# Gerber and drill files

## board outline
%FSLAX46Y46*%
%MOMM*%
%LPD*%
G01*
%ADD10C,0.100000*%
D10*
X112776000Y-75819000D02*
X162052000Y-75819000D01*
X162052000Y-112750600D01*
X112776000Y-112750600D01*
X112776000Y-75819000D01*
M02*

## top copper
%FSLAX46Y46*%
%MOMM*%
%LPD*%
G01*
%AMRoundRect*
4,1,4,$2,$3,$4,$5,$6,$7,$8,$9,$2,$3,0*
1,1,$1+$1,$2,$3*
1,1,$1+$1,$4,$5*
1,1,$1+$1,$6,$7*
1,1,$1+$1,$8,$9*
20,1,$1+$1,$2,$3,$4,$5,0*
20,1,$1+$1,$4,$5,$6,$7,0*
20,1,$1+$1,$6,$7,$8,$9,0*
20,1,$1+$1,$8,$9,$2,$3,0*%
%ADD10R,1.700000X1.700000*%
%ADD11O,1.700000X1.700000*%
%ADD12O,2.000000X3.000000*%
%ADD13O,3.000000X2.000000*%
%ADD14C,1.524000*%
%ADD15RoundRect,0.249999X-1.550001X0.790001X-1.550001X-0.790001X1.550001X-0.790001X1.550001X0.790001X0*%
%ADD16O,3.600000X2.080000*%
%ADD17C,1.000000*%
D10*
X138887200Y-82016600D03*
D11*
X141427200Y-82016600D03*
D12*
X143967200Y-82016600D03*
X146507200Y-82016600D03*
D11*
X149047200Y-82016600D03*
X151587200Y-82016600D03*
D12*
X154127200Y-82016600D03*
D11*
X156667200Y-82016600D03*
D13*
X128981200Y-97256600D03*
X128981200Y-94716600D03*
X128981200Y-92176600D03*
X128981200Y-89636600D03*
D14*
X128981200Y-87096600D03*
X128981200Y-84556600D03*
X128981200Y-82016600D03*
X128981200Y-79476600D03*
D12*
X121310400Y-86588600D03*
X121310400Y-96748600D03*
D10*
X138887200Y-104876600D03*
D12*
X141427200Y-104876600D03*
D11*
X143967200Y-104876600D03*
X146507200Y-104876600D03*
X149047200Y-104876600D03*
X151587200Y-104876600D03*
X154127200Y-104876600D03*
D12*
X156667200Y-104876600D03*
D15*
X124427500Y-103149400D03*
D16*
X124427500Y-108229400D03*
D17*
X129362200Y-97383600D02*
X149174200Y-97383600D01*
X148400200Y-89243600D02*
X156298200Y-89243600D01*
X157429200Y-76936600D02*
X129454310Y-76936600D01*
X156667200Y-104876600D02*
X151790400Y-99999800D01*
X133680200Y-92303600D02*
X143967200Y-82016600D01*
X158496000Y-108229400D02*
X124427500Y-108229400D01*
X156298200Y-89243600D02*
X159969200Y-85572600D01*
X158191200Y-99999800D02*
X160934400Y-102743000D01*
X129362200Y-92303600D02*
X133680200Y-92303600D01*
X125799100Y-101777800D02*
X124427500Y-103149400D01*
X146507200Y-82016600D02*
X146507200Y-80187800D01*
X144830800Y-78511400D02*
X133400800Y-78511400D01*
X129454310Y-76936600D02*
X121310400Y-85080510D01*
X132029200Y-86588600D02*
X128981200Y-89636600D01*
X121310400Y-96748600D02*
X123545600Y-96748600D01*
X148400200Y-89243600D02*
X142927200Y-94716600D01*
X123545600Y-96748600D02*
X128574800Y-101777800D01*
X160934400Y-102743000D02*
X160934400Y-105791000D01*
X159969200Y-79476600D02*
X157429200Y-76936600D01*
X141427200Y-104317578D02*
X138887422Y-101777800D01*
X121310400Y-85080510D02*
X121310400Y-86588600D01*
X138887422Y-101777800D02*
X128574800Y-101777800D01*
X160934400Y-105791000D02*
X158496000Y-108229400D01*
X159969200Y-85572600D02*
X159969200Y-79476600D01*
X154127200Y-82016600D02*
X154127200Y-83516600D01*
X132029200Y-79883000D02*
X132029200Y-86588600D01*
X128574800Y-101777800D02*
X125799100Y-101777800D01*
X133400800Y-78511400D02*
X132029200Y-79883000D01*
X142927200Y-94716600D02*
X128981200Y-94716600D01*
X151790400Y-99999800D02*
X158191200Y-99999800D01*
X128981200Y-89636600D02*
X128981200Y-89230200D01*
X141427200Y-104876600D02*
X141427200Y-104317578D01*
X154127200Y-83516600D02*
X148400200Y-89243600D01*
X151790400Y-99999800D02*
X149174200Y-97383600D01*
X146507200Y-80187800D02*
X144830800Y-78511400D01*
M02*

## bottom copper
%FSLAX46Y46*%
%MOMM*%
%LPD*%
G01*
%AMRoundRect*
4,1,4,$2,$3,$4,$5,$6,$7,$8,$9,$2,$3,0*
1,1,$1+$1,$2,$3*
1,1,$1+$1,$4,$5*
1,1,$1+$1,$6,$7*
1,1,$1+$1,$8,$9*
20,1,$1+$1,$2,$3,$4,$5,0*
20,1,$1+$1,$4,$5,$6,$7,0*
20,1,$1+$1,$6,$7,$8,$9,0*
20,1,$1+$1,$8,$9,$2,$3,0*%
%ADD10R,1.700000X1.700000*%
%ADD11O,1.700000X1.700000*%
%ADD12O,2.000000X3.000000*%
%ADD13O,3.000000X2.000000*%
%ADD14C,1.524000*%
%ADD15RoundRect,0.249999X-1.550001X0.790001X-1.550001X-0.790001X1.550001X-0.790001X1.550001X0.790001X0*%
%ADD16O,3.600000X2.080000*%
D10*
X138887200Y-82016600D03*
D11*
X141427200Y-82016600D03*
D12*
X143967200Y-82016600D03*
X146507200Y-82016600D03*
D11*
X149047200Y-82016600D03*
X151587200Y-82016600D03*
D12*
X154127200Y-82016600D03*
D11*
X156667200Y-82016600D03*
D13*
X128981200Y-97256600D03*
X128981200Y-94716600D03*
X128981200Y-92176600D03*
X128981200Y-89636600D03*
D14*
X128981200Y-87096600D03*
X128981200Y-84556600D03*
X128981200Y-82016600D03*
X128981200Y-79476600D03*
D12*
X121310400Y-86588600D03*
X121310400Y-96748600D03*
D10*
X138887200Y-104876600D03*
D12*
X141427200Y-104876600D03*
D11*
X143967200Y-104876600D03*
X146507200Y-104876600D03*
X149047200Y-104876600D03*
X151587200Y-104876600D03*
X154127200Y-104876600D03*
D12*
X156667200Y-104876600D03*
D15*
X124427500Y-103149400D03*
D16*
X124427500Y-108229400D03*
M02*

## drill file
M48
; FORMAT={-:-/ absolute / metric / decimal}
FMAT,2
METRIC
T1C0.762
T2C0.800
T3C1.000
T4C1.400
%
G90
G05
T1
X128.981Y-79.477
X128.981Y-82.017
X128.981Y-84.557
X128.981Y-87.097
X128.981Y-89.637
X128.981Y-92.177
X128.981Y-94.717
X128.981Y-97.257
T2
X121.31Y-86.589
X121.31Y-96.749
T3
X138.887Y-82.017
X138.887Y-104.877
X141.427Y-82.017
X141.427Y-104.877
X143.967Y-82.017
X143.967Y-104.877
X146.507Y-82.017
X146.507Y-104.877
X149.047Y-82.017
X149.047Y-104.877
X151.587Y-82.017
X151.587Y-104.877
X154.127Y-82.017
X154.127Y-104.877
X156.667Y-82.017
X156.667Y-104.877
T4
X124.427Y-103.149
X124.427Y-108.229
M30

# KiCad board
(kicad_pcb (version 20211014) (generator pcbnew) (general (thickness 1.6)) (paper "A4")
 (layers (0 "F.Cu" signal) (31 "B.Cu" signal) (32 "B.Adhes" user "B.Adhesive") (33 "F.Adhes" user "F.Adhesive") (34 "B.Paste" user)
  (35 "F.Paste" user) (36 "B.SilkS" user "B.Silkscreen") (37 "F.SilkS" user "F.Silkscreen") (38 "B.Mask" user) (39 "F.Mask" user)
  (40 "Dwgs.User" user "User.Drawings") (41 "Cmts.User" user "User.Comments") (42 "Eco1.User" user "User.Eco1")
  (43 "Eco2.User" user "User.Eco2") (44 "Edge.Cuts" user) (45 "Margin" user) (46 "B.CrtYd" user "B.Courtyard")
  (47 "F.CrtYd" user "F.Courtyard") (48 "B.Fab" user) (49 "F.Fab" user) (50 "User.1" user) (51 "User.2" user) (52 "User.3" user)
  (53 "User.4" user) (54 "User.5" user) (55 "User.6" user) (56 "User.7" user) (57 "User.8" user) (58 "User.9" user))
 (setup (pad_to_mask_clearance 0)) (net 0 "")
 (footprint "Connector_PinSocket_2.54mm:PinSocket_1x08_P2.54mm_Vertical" (layer "F.Cu") (at 138.8872 82.0166 90)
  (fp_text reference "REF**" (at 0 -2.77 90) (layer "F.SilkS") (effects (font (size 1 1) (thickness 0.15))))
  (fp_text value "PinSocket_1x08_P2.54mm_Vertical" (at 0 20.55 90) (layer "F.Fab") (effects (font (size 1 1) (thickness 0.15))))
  (pad "1" thru_hole rect (at 0 0 90) (size 1.7 1.7) (drill 1) (layers *.Cu *.Mask))
  (pad "2" thru_hole oval (at 0 2.54 90) (size 1.7 1.7) (drill 1) (layers *.Cu *.Mask))
  (pad "3" thru_hole oval (at 0 5.08 90) (size 3 2) (drill 1) (layers *.Cu *.Mask))
  (pad "4" thru_hole oval (at 0 7.62 90) (size 3 2) (drill 1) (layers *.Cu *.Mask))
  (pad "5" thru_hole oval (at 0 10.16 90) (size 1.7 1.7) (drill 1) (layers *.Cu *.Mask))
  (pad "6" thru_hole oval (at 0 12.7 90) (size 1.7 1.7) (drill 1) (layers *.Cu *.Mask))
  (pad "7" thru_hole oval (at 0 15.24 90) (size 3 2) (drill 1) (layers *.Cu *.Mask))
  (pad "8" thru_hole oval (at 0 17.78 90) (size 1.7 1.7) (drill 1) (layers *.Cu *.Mask)))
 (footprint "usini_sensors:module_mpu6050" (layer "F.Cu") (at 128.9812 79.4766 180)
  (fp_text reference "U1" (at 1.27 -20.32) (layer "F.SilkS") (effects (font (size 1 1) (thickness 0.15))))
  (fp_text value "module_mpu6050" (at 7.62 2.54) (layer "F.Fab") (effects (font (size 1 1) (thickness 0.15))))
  (pad "1" thru_hole oval locked (at 0 -17.78 180) (size 3 2) (drill 0.762) (layers *.Cu *.Mask))
  (pad "2" thru_hole oval locked (at 0 -15.24 180) (size 3 2) (drill 0.762) (layers *.Cu *.Mask))
  (pad "3" thru_hole oval locked (at 0 -12.7 180) (size 3 2) (drill 0.762) (layers *.Cu *.Mask))
  (pad "4" thru_hole oval locked (at 0 -10.16 180) (size 3 2) (drill 0.762) (layers *.Cu *.Mask))
  (pad "5" thru_hole circle locked (at 0 -7.62 180) (size 1.524 1.524) (drill 0.762) (layers *.Cu *.Mask))
  (pad "6" thru_hole circle locked (at 0 -5.08 180) (size 1.524 1.524) (drill 0.762) (layers *.Cu *.Mask))
  (pad "7" thru_hole circle locked (at 0 -2.54 180) (size 1.524 1.524) (drill 0.762) (layers *.Cu *.Mask))
  (pad "8" thru_hole circle locked (at 0 0 180) (size 1.524 1.524) (drill 0.762) (layers *.Cu *.Mask)))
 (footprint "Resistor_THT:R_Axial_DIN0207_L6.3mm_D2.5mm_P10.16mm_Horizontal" (layer "F.Cu") (at 121.3104 86.5886 -90)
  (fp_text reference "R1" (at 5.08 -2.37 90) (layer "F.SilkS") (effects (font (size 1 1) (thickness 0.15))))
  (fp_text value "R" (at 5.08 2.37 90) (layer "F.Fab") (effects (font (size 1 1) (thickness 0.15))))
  (pad "1" thru_hole oval (at 0 0 270) (size 3 2) (drill 0.8) (layers *.Cu *.Mask))
  (pad "2" thru_hole oval (at 10.16 0 270) (size 3 2) (drill 0.8) (layers *.Cu *.Mask)))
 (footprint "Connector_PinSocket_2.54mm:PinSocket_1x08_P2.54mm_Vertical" (layer "F.Cu") (at 138.8872 104.8766 90)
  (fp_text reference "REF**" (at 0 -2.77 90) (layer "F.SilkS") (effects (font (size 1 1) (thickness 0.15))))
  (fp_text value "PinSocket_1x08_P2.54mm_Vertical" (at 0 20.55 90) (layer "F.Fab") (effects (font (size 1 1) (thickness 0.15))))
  (pad "1" thru_hole rect (at 0 0 90) (size 1.7 1.7) (drill 1) (layers *.Cu *.Mask))
  (pad "2" thru_hole oval (at 0 2.54 90) (size 3 2) (drill 1) (layers *.Cu *.Mask))
  (pad "3" thru_hole oval (at 0 5.08 90) (size 1.7 1.7) (drill 1) (layers *.Cu *.Mask))
  (pad "4" thru_hole oval (at 0 7.62 90) (size 1.7 1.7) (drill 1) (layers *.Cu *.Mask))
  (pad "5" thru_hole oval (at 0 10.16 90) (size 1.7 1.7) (drill 1) (layers *.Cu *.Mask))
  (pad "6" thru_hole oval (at 0 12.7 90) (size 1.7 1.7) (drill 1) (layers *.Cu *.Mask))
  (pad "7" thru_hole oval (at 0 15.24 90) (size 1.7 1.7) (drill 1) (layers *.Cu *.Mask))
  (pad "8" thru_hole oval (at 0 17.78 90) (size 3 2) (drill 1) (layers *.Cu *.Mask)))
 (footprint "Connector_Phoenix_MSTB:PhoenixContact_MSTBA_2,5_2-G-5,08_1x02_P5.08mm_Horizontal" (layer "F.Cu") (at 124.4275 103.1494 -90)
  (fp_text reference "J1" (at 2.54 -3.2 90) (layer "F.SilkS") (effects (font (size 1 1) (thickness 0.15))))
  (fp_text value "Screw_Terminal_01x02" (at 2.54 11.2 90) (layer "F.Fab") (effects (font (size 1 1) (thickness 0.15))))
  (pad "1" thru_hole roundrect (at 0 0 270) (size 2.08 3.6) (drill 1.4) (layers *.Cu *.Mask) (roundrect_rratio 0.120192))
  (pad "2" thru_hole oval (at 5.08 0 270) (size 2.08 3.6) (drill 1.4) (layers *.Cu *.Mask)))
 (gr_rect (start 112.776 112.7506) (end 162.052 75.819) (layer "Edge.Cuts") (width 0.1) (fill none))
 (segment (start 129.3622 97.3836) (end 149.1742 97.3836) (width 1) (layer "F.Cu") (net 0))
 (segment (start 148.4002 89.2436) (end 156.2982 89.2436) (width 1) (layer "F.Cu") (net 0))
 (segment (start 157.4292 76.9366) (end 129.45431 76.9366) (width 1) (layer "F.Cu") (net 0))
 (segment (start 156.6672 104.8766) (end 151.7904 99.9998) (width 1) (layer "F.Cu") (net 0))
 (segment (start 133.6802 92.3036) (end 143.9672 82.0166) (width 1) (layer "F.Cu") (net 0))
 (segment (start 158.496 108.2294) (end 124.4275 108.2294) (width 1) (layer "F.Cu") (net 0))
 (segment (start 156.2982 89.2436) (end 159.9692 85.5726) (width 1) (layer "F.Cu") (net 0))
 (segment (start 158.1912 99.9998) (end 160.9344 102.743) (width 1) (layer "F.Cu") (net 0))
 (segment (start 129.3622 92.3036) (end 133.6802 92.3036) (width 1) (layer "F.Cu") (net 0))
 (segment (start 125.7991 101.7778) (end 124.4275 103.1494) (width 1) (layer "F.Cu") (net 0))
 (segment (start 146.5072 82.0166) (end 146.5072 80.1878) (width 1) (layer "F.Cu") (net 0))
 (segment (start 144.8308 78.5114) (end 133.4008 78.5114) (width 1) (layer "F.Cu") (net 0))
 (segment (start 129.45431 76.9366) (end 121.3104 85.08051) (width 1) (layer "F.Cu") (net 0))
 (segment (start 132.0292 86.5886) (end 128.9812 89.6366) (width 1) (layer "F.Cu") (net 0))
 (segment (start 121.3104 96.7486) (end 123.5456 96.7486) (width 1) (layer "F.Cu") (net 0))
 (segment (start 148.4002 89.2436) (end 142.9272 94.7166) (width 1) (layer "F.Cu") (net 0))
 (segment (start 123.5456 96.7486) (end 128.5748 101.7778) (width 1) (layer "F.Cu") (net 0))
 (segment (start 160.9344 102.743) (end 160.9344 105.791) (width 1) (layer "F.Cu") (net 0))
 (segment (start 159.9692 79.4766) (end 157.4292 76.9366) (width 1) (layer "F.Cu") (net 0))
 (segment (start 141.4272 104.317578) (end 138.887422 101.7778) (width 1) (layer "F.Cu") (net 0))
 (segment (start 121.3104 85.08051) (end 121.3104 86.5886) (width 1) (layer "F.Cu") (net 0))
 (segment (start 138.887422 101.7778) (end 128.5748 101.7778) (width 1) (layer "F.Cu") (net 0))
 (segment (start 160.9344 105.791) (end 158.496 108.2294) (width 1) (layer "F.Cu") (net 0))
 (segment (start 159.9692 85.5726) (end 159.9692 79.4766) (width 1) (layer "F.Cu") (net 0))
 (segment (start 154.1272 82.0166) (end 154.1272 83.5166) (width 1) (layer "F.Cu") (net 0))
 (segment (start 132.0292 79.883) (end 132.0292 86.5886) (width 1) (layer "F.Cu") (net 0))
 (segment (start 128.5748 101.7778) (end 125.7991 101.7778) (width 1) (layer "F.Cu") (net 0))
 (segment (start 133.4008 78.5114) (end 132.0292 79.883) (width 1) (layer "F.Cu") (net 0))
 (segment (start 142.9272 94.7166) (end 128.9812 94.7166) (width 1) (layer "F.Cu") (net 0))
 (segment (start 151.7904 99.9998) (end 158.1912 99.9998) (width 1) (layer "F.Cu") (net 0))
 (segment (start 128.9812 89.6366) (end 128.9812 89.2302) (width 1) (layer "F.Cu") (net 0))
 (segment (start 141.4272 104.8766) (end 141.4272 104.317578) (width 1) (layer "F.Cu") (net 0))
 (segment (start 154.1272 83.5166) (end 148.4002 89.2436) (width 1) (layer "F.Cu") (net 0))
 (segment (start 151.7904 99.9998) (end 149.1742 97.3836) (width 1) (layer "F.Cu") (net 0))
 (segment (start 146.5072 80.1878) (end 144.8308 78.5114) (width 1) (layer "F.Cu") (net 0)))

